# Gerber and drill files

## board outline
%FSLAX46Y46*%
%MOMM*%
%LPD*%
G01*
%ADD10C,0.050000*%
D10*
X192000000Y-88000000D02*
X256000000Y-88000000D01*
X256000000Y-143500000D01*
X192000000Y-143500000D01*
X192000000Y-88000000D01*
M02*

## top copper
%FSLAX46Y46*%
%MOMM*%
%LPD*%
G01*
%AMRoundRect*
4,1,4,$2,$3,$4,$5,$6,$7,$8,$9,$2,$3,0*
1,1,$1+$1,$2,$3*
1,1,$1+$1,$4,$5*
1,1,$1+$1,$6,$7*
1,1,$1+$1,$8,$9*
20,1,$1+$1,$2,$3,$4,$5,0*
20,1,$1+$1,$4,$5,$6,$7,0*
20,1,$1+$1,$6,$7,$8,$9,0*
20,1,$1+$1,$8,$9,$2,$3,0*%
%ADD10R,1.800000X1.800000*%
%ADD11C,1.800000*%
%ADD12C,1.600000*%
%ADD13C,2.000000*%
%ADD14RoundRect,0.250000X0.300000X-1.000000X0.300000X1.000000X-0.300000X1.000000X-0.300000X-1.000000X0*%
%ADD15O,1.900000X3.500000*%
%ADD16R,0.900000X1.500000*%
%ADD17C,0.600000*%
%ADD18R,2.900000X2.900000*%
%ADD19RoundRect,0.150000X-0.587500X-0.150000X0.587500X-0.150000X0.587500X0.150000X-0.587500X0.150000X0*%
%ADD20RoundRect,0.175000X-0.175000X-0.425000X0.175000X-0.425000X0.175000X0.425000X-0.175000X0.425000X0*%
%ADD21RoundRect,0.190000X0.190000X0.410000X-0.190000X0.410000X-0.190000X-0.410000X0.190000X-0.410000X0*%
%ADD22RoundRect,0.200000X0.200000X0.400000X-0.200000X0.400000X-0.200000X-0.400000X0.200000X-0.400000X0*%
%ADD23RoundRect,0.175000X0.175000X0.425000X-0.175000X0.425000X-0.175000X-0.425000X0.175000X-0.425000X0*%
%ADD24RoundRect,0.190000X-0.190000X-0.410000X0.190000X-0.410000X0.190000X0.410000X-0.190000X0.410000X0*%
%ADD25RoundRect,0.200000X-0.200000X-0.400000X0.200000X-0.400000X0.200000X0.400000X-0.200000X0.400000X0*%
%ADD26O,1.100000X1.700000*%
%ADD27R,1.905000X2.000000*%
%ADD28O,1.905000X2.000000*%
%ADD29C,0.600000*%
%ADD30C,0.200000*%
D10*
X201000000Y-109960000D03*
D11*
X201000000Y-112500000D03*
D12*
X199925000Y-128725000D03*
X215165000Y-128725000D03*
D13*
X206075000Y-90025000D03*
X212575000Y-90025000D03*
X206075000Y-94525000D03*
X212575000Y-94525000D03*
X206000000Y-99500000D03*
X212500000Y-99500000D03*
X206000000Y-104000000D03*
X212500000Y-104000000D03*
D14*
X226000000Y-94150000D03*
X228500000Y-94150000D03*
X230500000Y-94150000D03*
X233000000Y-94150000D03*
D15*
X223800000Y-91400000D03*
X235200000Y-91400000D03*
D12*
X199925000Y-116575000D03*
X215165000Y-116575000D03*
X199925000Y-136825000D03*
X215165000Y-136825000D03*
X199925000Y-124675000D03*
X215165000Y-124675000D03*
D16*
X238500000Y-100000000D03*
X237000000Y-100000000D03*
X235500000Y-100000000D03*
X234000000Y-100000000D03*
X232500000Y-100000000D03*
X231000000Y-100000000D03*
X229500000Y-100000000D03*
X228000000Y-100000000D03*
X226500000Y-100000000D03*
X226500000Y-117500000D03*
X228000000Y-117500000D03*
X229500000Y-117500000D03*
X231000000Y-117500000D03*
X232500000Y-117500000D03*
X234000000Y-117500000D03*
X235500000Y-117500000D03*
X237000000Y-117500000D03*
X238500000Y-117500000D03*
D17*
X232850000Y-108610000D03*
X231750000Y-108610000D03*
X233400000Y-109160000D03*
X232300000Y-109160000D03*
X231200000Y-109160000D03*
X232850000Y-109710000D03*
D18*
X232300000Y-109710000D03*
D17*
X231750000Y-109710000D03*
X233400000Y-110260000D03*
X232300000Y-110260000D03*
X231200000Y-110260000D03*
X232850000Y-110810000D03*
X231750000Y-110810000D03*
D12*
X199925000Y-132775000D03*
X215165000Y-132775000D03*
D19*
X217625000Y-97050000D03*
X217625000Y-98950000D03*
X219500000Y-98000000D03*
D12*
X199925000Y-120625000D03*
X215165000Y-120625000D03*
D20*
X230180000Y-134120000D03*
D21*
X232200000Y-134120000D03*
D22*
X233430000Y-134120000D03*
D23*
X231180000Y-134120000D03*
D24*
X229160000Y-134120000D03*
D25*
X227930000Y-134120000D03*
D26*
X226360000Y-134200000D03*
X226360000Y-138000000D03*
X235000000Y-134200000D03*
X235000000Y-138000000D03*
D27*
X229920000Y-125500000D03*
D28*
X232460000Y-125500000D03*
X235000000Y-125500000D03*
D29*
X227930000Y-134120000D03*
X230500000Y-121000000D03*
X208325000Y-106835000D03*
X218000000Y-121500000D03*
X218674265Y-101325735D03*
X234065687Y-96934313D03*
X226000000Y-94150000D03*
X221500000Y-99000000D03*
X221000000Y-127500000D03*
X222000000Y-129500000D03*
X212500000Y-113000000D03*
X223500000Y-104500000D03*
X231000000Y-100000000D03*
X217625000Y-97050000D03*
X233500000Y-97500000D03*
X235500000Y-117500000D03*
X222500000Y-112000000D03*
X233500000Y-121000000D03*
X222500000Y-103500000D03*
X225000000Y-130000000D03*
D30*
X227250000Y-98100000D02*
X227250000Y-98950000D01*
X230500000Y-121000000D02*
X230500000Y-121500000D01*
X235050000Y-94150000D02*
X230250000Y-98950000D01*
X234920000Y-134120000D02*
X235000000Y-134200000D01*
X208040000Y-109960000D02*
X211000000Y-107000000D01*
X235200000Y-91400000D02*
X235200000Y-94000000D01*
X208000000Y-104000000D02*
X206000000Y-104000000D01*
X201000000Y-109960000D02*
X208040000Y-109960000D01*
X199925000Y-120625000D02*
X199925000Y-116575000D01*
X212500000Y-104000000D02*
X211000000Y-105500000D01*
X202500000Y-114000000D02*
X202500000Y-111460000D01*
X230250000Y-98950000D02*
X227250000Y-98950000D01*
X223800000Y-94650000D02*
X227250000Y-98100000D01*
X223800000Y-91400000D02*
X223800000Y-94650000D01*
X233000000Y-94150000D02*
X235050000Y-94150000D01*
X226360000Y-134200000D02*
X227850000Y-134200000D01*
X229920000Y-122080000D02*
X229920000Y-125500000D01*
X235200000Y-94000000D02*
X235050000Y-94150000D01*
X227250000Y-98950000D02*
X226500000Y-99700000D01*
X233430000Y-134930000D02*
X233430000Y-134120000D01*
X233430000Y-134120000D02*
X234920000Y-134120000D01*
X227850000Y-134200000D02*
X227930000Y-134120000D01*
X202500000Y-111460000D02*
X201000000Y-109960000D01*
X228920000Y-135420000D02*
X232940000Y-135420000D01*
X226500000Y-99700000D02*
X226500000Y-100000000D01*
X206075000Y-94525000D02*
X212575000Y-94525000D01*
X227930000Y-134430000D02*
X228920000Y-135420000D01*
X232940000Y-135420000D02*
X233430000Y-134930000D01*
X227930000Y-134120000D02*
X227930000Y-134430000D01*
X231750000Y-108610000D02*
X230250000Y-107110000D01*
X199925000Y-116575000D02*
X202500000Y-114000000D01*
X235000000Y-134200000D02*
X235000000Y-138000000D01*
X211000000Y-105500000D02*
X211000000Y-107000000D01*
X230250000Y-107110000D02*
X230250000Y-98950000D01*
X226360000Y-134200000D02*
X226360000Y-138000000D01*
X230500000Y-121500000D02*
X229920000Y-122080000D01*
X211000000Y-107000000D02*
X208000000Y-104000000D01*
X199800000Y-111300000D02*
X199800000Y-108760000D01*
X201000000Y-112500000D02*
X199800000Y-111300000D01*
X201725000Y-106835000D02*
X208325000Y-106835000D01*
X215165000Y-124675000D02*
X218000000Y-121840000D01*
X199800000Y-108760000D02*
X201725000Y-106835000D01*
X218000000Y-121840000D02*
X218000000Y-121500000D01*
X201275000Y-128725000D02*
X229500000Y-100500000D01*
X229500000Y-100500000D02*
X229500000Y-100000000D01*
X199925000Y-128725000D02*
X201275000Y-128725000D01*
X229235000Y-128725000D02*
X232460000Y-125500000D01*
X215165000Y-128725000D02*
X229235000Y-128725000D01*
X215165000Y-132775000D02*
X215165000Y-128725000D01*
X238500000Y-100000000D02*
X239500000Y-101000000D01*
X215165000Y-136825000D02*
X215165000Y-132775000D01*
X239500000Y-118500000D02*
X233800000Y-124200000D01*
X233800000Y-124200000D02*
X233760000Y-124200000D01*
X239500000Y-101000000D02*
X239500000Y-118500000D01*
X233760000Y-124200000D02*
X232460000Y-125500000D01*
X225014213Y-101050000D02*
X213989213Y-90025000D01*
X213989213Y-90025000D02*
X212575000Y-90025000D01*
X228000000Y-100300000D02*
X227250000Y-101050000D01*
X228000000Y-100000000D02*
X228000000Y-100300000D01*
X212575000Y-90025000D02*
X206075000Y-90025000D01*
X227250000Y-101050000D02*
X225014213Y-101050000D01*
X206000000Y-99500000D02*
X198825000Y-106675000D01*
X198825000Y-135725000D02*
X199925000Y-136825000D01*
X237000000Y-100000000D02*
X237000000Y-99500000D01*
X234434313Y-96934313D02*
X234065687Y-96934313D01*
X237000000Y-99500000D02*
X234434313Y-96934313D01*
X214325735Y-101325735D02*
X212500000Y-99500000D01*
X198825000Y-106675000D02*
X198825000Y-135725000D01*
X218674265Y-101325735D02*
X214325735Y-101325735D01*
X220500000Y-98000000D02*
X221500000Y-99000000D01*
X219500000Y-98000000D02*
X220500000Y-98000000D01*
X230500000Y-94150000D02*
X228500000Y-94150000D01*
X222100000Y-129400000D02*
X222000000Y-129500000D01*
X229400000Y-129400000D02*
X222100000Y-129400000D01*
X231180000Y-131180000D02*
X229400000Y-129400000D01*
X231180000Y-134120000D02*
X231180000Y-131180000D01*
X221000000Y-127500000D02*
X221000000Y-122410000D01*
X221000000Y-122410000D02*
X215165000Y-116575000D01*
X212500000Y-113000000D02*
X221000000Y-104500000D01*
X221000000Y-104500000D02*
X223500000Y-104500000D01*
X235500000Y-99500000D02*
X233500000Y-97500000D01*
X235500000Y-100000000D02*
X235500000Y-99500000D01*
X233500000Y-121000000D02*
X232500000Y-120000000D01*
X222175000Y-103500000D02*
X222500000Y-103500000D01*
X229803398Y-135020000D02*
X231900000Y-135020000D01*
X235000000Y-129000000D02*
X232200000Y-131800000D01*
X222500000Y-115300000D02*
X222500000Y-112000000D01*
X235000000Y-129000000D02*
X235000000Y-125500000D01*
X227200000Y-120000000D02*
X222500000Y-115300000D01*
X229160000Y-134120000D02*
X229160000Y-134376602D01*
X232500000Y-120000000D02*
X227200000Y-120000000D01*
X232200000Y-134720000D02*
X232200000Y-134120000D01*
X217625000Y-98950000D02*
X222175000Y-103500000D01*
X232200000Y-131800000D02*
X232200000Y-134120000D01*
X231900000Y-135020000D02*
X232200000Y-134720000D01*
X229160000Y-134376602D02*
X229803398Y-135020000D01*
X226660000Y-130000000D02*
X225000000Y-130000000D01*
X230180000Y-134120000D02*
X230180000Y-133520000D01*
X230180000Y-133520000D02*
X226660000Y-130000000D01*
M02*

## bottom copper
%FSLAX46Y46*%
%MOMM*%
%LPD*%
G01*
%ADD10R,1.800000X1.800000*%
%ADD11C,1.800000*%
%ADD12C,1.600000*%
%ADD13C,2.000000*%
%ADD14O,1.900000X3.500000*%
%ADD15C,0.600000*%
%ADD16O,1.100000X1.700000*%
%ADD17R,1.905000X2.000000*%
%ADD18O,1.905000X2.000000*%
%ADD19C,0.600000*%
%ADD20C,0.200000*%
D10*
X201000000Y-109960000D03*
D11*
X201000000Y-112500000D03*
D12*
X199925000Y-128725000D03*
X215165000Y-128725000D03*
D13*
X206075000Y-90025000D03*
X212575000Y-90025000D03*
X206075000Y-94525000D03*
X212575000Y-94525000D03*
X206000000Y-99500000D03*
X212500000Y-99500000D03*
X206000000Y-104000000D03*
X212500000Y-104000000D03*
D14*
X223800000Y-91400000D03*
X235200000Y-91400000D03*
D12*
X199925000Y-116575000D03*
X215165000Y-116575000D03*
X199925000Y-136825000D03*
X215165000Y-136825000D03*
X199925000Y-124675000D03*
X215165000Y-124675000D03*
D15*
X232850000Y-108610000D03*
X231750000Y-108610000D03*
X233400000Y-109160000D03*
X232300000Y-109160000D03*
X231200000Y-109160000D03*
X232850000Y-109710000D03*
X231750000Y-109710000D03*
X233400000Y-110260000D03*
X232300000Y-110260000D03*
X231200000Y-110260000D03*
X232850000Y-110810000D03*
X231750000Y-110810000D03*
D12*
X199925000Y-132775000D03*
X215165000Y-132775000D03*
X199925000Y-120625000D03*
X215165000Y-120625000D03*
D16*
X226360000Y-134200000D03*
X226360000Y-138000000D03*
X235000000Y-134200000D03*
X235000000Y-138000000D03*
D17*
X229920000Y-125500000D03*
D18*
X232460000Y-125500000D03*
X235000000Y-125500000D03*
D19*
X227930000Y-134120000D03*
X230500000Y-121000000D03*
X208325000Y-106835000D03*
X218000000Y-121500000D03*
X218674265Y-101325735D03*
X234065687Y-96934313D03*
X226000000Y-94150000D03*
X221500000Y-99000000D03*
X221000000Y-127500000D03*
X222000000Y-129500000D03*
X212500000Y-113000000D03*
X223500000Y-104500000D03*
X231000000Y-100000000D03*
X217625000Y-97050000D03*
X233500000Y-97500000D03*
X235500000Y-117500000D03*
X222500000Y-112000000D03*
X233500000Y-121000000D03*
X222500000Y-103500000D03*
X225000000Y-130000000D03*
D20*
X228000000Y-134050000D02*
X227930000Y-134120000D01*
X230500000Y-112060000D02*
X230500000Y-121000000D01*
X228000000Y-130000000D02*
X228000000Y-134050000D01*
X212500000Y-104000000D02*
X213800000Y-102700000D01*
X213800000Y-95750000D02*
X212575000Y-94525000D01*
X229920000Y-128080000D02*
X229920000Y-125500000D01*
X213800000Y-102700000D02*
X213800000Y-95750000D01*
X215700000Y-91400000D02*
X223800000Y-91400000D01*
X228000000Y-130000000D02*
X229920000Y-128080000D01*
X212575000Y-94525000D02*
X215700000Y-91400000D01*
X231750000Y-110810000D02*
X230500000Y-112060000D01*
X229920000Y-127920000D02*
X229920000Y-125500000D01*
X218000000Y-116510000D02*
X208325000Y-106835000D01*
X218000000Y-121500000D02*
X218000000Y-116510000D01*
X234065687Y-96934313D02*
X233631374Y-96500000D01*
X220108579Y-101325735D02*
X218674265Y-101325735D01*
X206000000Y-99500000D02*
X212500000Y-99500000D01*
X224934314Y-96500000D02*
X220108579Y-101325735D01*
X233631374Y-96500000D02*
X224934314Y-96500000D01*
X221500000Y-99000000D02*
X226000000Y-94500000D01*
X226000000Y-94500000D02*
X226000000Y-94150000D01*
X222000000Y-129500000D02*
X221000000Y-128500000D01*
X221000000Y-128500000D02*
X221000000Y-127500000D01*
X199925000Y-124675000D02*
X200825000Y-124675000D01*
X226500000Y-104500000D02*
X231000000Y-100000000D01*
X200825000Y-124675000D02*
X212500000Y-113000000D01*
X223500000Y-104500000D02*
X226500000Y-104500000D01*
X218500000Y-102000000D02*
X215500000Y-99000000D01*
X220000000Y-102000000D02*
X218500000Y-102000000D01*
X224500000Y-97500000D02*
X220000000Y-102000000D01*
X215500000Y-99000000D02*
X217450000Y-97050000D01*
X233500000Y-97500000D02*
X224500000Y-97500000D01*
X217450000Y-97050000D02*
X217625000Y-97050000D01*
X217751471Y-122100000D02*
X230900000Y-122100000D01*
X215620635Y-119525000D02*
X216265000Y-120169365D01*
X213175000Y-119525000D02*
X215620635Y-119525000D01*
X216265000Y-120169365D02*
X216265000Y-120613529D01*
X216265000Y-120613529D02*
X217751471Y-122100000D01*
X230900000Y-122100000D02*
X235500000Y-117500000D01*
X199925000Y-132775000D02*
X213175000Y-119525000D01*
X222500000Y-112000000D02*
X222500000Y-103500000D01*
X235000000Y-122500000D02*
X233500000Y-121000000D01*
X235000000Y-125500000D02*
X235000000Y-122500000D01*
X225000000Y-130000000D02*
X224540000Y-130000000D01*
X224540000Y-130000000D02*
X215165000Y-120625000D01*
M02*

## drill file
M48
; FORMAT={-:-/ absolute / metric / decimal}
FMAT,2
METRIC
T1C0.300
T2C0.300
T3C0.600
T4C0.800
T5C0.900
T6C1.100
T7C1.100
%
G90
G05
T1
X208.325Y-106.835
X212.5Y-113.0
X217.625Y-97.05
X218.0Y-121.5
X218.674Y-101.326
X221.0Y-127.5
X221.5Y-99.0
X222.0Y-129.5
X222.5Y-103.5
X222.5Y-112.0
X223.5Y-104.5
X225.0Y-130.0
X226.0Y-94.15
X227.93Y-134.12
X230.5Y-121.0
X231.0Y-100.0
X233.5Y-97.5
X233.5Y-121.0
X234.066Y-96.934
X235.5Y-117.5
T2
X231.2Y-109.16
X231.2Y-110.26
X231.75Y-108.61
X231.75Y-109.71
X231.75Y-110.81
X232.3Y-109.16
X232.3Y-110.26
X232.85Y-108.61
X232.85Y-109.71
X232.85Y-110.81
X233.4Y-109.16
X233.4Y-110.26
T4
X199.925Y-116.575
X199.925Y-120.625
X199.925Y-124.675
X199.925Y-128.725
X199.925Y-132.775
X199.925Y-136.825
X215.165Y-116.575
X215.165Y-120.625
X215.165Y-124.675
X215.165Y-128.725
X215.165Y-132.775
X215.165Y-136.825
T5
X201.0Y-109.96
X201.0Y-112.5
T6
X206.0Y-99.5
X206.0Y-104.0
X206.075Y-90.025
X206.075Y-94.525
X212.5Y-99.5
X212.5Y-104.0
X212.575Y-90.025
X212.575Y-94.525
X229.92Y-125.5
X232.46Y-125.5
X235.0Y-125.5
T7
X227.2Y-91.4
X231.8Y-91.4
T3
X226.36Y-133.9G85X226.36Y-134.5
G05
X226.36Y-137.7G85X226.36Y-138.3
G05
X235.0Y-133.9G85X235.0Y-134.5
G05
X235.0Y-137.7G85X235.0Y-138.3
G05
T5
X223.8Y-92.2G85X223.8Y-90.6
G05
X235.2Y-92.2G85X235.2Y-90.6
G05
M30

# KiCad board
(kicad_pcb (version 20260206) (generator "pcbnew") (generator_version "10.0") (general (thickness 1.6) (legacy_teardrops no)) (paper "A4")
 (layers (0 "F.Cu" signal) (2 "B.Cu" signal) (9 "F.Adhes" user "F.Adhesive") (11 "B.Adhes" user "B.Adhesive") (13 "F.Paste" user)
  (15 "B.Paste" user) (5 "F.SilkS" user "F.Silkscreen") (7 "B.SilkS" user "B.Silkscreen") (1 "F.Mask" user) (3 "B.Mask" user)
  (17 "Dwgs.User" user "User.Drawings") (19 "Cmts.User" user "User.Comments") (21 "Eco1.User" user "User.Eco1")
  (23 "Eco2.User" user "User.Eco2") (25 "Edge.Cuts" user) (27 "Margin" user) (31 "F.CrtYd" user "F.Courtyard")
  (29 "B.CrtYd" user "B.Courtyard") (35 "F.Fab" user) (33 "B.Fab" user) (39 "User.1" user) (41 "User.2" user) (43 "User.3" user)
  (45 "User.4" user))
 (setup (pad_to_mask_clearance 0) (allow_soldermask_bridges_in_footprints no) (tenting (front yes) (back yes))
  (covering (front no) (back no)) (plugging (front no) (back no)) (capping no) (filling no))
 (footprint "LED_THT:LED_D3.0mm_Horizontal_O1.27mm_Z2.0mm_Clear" (layer "F.Cu") (at 201 109.96 -90)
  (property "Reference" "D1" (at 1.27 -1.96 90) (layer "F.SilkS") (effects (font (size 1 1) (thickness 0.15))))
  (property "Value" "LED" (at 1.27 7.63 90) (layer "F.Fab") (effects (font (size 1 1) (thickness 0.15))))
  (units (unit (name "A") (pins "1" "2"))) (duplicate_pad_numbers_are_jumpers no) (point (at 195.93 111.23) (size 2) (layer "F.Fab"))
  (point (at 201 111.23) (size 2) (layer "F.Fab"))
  (pad "1" thru_hole rect (at 0 0 270) (size 1.8 1.8) (drill 0.9) (layers "*.Cu" "*.Mask") (remove_unused_layers no) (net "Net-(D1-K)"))
  (pad "2" thru_hole circle (at 2.54 0 270) (size 1.8 1.8) (drill 0.9) (layers "*.Cu" "*.Mask") (remove_unused_layers no) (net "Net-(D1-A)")))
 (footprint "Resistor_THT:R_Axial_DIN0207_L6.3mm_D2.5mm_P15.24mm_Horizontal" (layer "F.Cu") (at 199.925 128.725)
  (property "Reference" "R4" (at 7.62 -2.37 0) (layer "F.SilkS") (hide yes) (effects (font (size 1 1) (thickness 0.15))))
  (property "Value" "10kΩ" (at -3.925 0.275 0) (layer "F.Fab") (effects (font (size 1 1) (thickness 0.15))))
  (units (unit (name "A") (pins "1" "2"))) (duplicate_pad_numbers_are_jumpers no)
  (pad "1" thru_hole circle (at 0 0) (size 1.6 1.6) (drill 0.8) (layers "*.Cu" "*.Mask") (remove_unused_layers no) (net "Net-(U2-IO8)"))
  (pad "2" thru_hole circle (at 15.24 0) (size 1.6 1.6) (drill 0.8) (layers "*.Cu" "*.Mask") (remove_unused_layers no) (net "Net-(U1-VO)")))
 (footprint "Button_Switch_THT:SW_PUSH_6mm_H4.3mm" (layer "F.Cu") (at 206.075 90.025)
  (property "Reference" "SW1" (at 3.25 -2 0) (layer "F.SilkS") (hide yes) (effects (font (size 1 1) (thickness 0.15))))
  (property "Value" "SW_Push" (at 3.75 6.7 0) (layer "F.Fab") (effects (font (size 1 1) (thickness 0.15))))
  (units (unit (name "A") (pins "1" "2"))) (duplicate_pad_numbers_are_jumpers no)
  (pad "1" thru_hole circle (at 0 0 90) (size 2 2) (drill 1.1) (layers "*.Cu" "*.Mask") (remove_unused_layers no) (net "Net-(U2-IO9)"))
  (pad "1" thru_hole circle (at 6.5 0 90) (size 2 2) (drill 1.1) (layers "*.Cu" "*.Mask") (remove_unused_layers no) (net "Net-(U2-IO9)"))
  (pad "2" thru_hole circle (at 0 4.5 90) (size 2 2) (drill 1.1) (layers "*.Cu" "*.Mask") (remove_unused_layers no) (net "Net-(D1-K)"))
  (pad "2" thru_hole circle (at 6.5 4.5 90) (size 2 2) (drill 1.1) (layers "*.Cu" "*.Mask") (remove_unused_layers no) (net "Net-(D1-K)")))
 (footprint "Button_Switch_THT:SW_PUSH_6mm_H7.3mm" (layer "F.Cu") (at 206 99.5)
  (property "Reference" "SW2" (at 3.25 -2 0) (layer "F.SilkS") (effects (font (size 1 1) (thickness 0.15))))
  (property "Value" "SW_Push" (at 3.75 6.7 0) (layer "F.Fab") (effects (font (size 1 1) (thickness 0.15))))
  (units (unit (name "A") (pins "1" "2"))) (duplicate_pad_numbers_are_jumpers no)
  (pad "1" thru_hole circle (at 0 0 90) (size 2 2) (drill 1.1) (layers "*.Cu" "*.Mask") (remove_unused_layers no) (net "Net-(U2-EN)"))
  (pad "1" thru_hole circle (at 6.5 0 90) (size 2 2) (drill 1.1) (layers "*.Cu" "*.Mask") (remove_unused_layers no) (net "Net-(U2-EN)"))
  (pad "2" thru_hole circle (at 0 4.5 90) (size 2 2) (drill 1.1) (layers "*.Cu" "*.Mask") (remove_unused_layers no) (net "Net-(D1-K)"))
  (pad "2" thru_hole circle (at 6.5 4.5 90) (size 2 2) (drill 1.1) (layers "*.Cu" "*.Mask") (remove_unused_layers no) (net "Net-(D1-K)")))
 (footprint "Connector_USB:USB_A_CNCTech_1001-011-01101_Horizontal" (layer "F.Cu") (at 229.5 84.5 90)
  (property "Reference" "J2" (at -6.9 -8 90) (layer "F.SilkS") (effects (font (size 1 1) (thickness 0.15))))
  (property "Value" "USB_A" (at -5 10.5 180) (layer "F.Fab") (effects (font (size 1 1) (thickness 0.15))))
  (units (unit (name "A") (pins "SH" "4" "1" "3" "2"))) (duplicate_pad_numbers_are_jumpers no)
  (pad "" np_thru_hole circle (at -6.9 -2.3 90) (size 1.1 1.1) (drill 1.1) (layers "*.Cu" "*.Mask"))
  (pad "" np_thru_hole circle (at -6.9 2.3 90) (size 1.1 1.1) (drill 1.1) (layers "*.Cu" "*.Mask"))
  (pad "1" smd roundrect (at -9.65 -3.5 90) (size 2.5 1.1) (layers "F.Cu" "F.Mask" "F.Paste") (roundrect_rratio 0.2272727273)
   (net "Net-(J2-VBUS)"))
  (pad "2" smd roundrect (at -9.65 -1 90) (size 2.5 1.1) (layers "F.Cu" "F.Mask" "F.Paste") (roundrect_rratio 0.2272727273)
   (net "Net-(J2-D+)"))
  (pad "3" smd roundrect (at -9.65 1 90) (size 2.5 1.1) (layers "F.Cu" "F.Mask" "F.Paste") (roundrect_rratio 0.2272727273)
   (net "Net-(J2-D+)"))
  (pad "4" smd roundrect (at -9.65 3.5 90) (size 2.5 1.1) (layers "F.Cu" "F.Mask" "F.Paste") (roundrect_rratio 0.2272727273)
   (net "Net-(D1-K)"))
  (pad "SH" thru_hole oval (at -6.9 -5.7 90) (size 3.5 1.9) (drill oval 2.5 0.9) (layers "*.Cu" "*.Mask") (remove_unused_layers no)
   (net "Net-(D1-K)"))
  (pad "SH" thru_hole oval (at -6.9 5.7 90) (size 3.5 1.9) (drill oval 2.5 0.9) (layers "*.Cu" "*.Mask") (remove_unused_layers no)
   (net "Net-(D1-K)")))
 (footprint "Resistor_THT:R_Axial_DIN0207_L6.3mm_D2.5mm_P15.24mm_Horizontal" (layer "F.Cu") (at 199.925 116.575)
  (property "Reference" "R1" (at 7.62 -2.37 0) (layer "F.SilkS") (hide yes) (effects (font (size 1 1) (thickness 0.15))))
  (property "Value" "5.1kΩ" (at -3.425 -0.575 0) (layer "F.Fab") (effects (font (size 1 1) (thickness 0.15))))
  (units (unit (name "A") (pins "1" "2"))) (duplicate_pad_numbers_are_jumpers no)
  (pad "1" thru_hole circle (at 0 0) (size 1.6 1.6) (drill 0.8) (layers "*.Cu" "*.Mask") (remove_unused_layers no) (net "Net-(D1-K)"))
  (pad "2" thru_hole circle (at 15.24 0) (size 1.6 1.6) (drill 0.8) (layers "*.Cu" "*.Mask") (remove_unused_layers no) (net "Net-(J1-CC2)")))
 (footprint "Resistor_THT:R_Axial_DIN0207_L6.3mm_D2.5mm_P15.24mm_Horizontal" (layer "F.Cu") (at 199.925 136.825)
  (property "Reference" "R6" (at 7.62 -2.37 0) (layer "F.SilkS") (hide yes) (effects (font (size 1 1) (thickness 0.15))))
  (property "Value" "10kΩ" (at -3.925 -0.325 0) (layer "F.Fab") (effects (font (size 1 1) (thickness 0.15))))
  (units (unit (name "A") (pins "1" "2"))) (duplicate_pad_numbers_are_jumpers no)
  (pad "1" thru_hole circle (at 0 0) (size 1.6 1.6) (drill 0.8) (layers "*.Cu" "*.Mask") (remove_unused_layers no) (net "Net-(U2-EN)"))
  (pad "2" thru_hole circle (at 15.24 0) (size 1.6 1.6) (drill 0.8) (layers "*.Cu" "*.Mask") (remove_unused_layers no) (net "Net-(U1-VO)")))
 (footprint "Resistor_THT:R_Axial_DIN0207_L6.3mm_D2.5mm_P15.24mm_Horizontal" (layer "F.Cu") (at 199.925 124.675)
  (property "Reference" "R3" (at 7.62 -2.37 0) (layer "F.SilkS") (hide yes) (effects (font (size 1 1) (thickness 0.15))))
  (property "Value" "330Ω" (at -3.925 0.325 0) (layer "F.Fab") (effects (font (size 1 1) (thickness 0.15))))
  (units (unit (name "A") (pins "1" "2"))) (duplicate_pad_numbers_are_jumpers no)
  (pad "1" thru_hole circle (at 0 0) (size 1.6 1.6) (drill 0.8) (layers "*.Cu" "*.Mask") (remove_unused_layers no) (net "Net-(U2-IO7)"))
  (pad "2" thru_hole circle (at 15.24 0) (size 1.6 1.6) (drill 0.8) (layers "*.Cu" "*.Mask") (remove_unused_layers no) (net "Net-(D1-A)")))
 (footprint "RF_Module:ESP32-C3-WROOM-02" (layer "F.Cu") (at 232.5 108.75 -90)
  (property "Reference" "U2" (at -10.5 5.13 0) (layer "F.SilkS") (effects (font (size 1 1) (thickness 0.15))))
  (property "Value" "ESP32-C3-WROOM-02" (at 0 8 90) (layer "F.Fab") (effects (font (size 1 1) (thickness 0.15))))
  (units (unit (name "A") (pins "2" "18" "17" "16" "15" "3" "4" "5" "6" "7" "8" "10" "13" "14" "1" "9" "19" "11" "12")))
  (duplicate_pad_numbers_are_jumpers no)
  (pad "" smd rect (at -0.14 -0.9 270) (size 0.7 0.7) (layers "F.Paste"))
  (pad "" smd rect (at -0.14 0.2 270) (size 0.7 0.7) (layers "F.Paste"))
  (pad "" smd rect (at -0.14 1.3 270) (size 0.7 0.7) (layers "F.Paste"))
  (pad "" smd rect (at 0.96 -0.9 270) (size 0.7 0.7) (layers "F.Paste"))
  (pad "" smd rect (at 0.96 0.2 270) (size 0.7 0.7) (layers "F.Paste"))
  (pad "" smd rect (at 0.96 1.3 270) (size 0.7 0.7) (layers "F.Paste"))
  (pad "" smd rect (at 2.06 -0.9 270) (size 0.7 0.7) (layers "F.Paste"))
  (pad "" smd rect (at 2.06 0.2 270) (size 0.7 0.7) (layers "F.Paste"))
  (pad "" smd rect (at 2.06 1.3 270) (size 0.7 0.7) (layers "F.Paste"))
  (pad "1" smd rect (at -8.75 -6 270) (size 1.5 0.9) (layers "F.Cu" "F.Mask" "F.Paste") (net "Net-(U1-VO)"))
  (pad "2" smd rect (at -8.75 -4.5 270) (size 1.5 0.9) (layers "F.Cu" "F.Mask" "F.Paste") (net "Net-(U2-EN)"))
  (pad "3" smd rect (at -8.75 -3 270) (size 1.5 0.9) (layers "F.Cu" "F.Mask" "F.Paste") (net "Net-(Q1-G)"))
  (pad "4" smd rect (at -8.75 -1.5 270) (size 1.5 0.9) (layers "F.Cu" "F.Mask" "F.Paste") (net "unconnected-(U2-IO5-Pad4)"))
  (pad "5" smd rect (at -8.75 0 270) (size 1.5 0.9) (layers "F.Cu" "F.Mask" "F.Paste") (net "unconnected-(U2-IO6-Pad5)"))
  (pad "6" smd rect (at -8.75 1.5 270) (size 1.5 0.9) (layers "F.Cu" "F.Mask" "F.Paste") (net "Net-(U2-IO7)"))
  (pad "7" smd rect (at -8.75 3 270) (size 1.5 0.9) (layers "F.Cu" "F.Mask" "F.Paste") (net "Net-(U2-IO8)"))
  (pad "8" smd rect (at -8.75 4.5 270) (size 1.5 0.9) (layers "F.Cu" "F.Mask" "F.Paste") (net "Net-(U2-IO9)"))
  (pad "9" smd rect (at -8.75 6 270) (size 1.5 0.9) (layers "F.Cu" "F.Mask" "F.Paste") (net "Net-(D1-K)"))
  (pad "10" smd rect (at 8.75 6 270) (size 1.5 0.9) (layers "F.Cu" "F.Mask" "F.Paste") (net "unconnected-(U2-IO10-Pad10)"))
  (pad "11" smd rect (at 8.75 4.5 270) (size 1.5 0.9) (layers "F.Cu" "F.Mask" "F.Paste") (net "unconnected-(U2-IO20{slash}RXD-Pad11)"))
  (pad "12" smd rect (at 8.75 3 270) (size 1.5 0.9) (layers "F.Cu" "F.Mask" "F.Paste") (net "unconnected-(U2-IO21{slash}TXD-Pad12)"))
  (pad "13" smd rect (at 8.75 1.5 270) (size 1.5 0.9) (layers "F.Cu" "F.Mask" "F.Paste") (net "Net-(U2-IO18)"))
  (pad "14" smd rect (at 8.75 0 270) (size 1.5 0.9) (layers "F.Cu" "F.Mask" "F.Paste") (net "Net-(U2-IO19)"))
  (pad "15" smd rect (at 8.75 -1.5 270) (size 1.5 0.9) (layers "F.Cu" "F.Mask" "F.Paste") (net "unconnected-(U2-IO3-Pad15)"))
  (pad "16" smd rect (at 8.75 -3 270) (size 1.5 0.9) (layers "F.Cu" "F.Mask" "F.Paste") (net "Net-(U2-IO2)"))
  (pad "17" smd rect (at 8.75 -4.5 270) (size 1.5 0.9) (layers "F.Cu" "F.Mask" "F.Paste") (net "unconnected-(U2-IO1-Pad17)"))
  (pad "18" smd rect (at 8.75 -6 270) (size 1.5 0.9) (layers "F.Cu" "F.Mask" "F.Paste") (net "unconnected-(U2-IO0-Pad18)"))
  (pad "19" thru_hole circle (at -0.14 -0.35 270) (size 0.6 0.6) (drill 0.3) (layers "*.Cu" "F.Mask") (remove_unused_layers no)
   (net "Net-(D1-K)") (zone_connect 2))
  (pad "19" thru_hole circle (at -0.14 0.75 270) (size 0.6 0.6) (drill 0.3) (layers "*.Cu" "F.Mask") (remove_unused_layers no)
   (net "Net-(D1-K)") (zone_connect 2))
  (pad "19" thru_hole circle (at 0.41 -0.9 270) (size 0.6 0.6) (drill 0.3) (layers "*.Cu" "F.Mask") (remove_unused_layers no)
   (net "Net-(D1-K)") (zone_connect 2))
  (pad "19" thru_hole circle (at 0.41 0.2 270) (size 0.6 0.6) (drill 0.3) (layers "*.Cu" "F.Mask") (remove_unused_layers no)
   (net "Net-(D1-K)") (zone_connect 2))
  (pad "19" thru_hole circle (at 0.41 1.3 270) (size 0.6 0.6) (drill 0.3) (layers "*.Cu" "F.Mask") (remove_unused_layers no)
   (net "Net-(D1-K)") (zone_connect 2))
  (pad "19" thru_hole circle (at 0.96 -0.35 270) (size 0.6 0.6) (drill 0.3) (layers "*.Cu" "F.Mask") (remove_unused_layers no)
   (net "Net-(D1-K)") (zone_connect 2))
  (pad "19" smd rect (at 0.96 0.2 270) (size 2.9 2.9) (layers "F.Cu" "F.Mask") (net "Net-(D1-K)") (zone_connect 2))
  (pad "19" thru_hole circle (at 0.96 0.75 270) (size 0.6 0.6) (drill 0.3) (layers "*.Cu" "F.Mask") (remove_unused_layers no)
   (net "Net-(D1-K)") (zone_connect 2))
  (pad "19" thru_hole circle (at 1.51 -0.9 270) (size 0.6 0.6) (drill 0.3) (layers "*.Cu" "F.Mask") (remove_unused_layers no)
   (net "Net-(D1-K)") (zone_connect 2))
  (pad "19" thru_hole circle (at 1.51 0.2 270) (size 0.6 0.6) (drill 0.3) (layers "*.Cu" "F.Mask") (remove_unused_layers no)
   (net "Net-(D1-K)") (zone_connect 2))
  (pad "19" thru_hole circle (at 1.51 1.3 270) (size 0.6 0.6) (drill 0.3) (layers "*.Cu" "F.Mask") (remove_unused_layers no)
   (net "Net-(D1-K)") (zone_connect 2))
  (pad "19" thru_hole circle (at 2.06 -0.35 270) (size 0.6 0.6) (drill 0.3) (layers "*.Cu" "F.Mask") (remove_unused_layers no)
   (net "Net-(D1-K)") (zone_connect 2))
  (pad "19" thru_hole circle (at 2.06 0.75 270) (size 0.6 0.6) (drill 0.3) (layers "*.Cu" "F.Mask") (remove_unused_layers no)
   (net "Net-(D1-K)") (zone_connect 2))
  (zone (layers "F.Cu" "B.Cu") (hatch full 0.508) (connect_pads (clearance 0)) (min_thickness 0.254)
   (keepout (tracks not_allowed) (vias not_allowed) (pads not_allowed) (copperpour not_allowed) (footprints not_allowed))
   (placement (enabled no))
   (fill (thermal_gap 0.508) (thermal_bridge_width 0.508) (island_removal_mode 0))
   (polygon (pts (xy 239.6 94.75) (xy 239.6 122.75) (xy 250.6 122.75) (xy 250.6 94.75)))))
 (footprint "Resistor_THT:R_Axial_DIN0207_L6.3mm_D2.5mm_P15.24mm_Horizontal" (layer "F.Cu") (at 199.925 132.775)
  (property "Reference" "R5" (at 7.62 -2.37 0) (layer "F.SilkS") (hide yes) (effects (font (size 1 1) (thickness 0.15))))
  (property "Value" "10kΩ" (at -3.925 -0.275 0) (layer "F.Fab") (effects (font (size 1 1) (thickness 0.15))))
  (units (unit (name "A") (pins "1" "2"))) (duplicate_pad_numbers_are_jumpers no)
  (pad "1" thru_hole circle (at 0 0) (size 1.6 1.6) (drill 0.8) (layers "*.Cu" "*.Mask") (remove_unused_layers no) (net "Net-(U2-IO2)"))
  (pad "2" thru_hole circle (at 15.24 0) (size 1.6 1.6) (drill 0.8) (layers "*.Cu" "*.Mask") (remove_unused_layers no) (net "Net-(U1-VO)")))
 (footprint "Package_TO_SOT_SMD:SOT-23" (layer "F.Cu") (at 218.5625 98)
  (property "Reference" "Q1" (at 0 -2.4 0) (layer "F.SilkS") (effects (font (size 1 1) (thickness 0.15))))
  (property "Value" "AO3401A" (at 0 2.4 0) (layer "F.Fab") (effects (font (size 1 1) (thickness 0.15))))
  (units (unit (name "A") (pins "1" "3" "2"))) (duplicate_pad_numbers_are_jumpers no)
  (pad "1" smd roundrect (at -0.9375 -0.95) (size 1.475 0.6) (layers "F.Cu" "F.Mask" "F.Paste") (roundrect_rratio 0.25) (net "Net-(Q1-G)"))
  (pad "2" smd roundrect (at -0.9375 0.95) (size 1.475 0.6) (layers "F.Cu" "F.Mask" "F.Paste") (roundrect_rratio 0.25) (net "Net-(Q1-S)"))
  (pad "3" smd roundrect (at 0.9375 0) (size 1.475 0.6) (layers "F.Cu" "F.Mask" "F.Paste") (roundrect_rratio 0.25) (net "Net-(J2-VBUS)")))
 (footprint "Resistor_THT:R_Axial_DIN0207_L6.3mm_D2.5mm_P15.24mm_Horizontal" (layer "F.Cu") (at 199.925 120.625)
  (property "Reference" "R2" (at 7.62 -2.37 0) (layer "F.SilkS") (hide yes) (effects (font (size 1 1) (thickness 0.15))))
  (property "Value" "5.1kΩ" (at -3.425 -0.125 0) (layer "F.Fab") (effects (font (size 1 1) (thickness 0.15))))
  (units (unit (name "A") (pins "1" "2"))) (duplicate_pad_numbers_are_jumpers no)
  (pad "1" thru_hole circle (at 0 0) (size 1.6 1.6) (drill 0.8) (layers "*.Cu" "*.Mask") (remove_unused_layers no) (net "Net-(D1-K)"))
  (pad "2" thru_hole circle (at 15.24 0) (size 1.6 1.6) (drill 0.8) (layers "*.Cu" "*.Mask") (remove_unused_layers no) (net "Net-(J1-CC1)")))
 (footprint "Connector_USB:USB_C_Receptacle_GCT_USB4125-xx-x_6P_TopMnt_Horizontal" (layer "F.Cu") (at 230.68 137.2)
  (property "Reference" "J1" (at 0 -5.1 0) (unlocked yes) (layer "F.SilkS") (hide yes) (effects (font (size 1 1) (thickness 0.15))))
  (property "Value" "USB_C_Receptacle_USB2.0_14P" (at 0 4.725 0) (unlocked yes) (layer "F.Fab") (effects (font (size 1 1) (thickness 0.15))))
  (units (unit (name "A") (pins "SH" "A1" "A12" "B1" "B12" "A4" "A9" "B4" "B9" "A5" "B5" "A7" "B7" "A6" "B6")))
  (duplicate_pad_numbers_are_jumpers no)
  (pad "A5" smd roundrect (at -0.5 -3.08) (size 0.7 1.2) (layers "F.Cu" "F.Mask" "F.Paste") (roundrect_rratio 0.25) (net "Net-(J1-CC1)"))
  (pad "A9" smd roundrect (at 1.52 -3.08 180) (size 0.76 1.2) (layers "F.Cu" "F.Mask" "F.Paste") (roundrect_rratio 0.25) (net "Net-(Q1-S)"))
  (pad "A12" smd roundrect (at 2.75 -3.08 180) (size 0.8 1.2) (layers "F.Cu" "F.Mask" "F.Paste") (roundrect_rratio 0.25) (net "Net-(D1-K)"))
  (pad "B5" smd roundrect (at 0.5 -3.08 180) (size 0.7 1.2) (layers "F.Cu" "F.Mask" "F.Paste") (roundrect_rratio 0.25) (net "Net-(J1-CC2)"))
  (pad "B9" smd roundrect (at -1.52 -3.08) (size 0.76 1.2) (layers "F.Cu" "F.Mask" "F.Paste") (roundrect_rratio 0.25) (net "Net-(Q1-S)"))
  (pad "B12" smd roundrect (at -2.75 -3.08) (size 0.8 1.2) (layers "F.Cu" "F.Mask" "F.Paste") (roundrect_rratio 0.25) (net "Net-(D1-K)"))
  (pad "SH" thru_hole oval (at -4.32 -3) (size 1.1 1.7) (drill oval 0.6 1.2) (layers "*.Cu" "*.Mask" "F.Paste") (remove_unused_layers no)
   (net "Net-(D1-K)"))
  (pad "SH" thru_hole oval (at -4.32 0.8) (size 1.1 1.7) (drill oval 0.6 1.2) (layers "*.Cu" "*.Mask" "F.Paste") (remove_unused_layers no)
   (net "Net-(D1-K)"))
  (pad "SH" thru_hole oval (at 4.32 -3) (size 1.1 1.7) (drill oval 0.6 1.2) (layers "*.Cu" "*.Mask" "F.Paste") (remove_unused_layers no)
   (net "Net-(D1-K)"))
  (pad "SH" thru_hole oval (at 4.32 0.8) (size 1.1 1.7) (drill oval 0.6 1.2) (layers "*.Cu" "*.Mask" "F.Paste") (remove_unused_layers no)
   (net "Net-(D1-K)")))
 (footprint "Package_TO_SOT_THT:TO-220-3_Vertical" (layer "F.Cu") (at 229.92 125.5)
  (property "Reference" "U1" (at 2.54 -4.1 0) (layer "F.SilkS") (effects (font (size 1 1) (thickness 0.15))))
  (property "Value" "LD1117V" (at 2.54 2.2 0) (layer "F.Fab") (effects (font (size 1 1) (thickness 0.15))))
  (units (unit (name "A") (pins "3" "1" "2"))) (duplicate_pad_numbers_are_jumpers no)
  (pad "1" thru_hole rect (at 0 0) (size 1.905 2) (drill 1.1) (layers "*.Cu" "*.Mask") (remove_unused_layers no) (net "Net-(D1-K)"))
  (pad "2" thru_hole oval (at 2.54 0) (size 1.905 2) (drill 1.1) (layers "*.Cu" "*.Mask") (remove_unused_layers no) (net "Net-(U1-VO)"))
  (pad "3" thru_hole oval (at 5.08 0) (size 1.905 2) (drill 1.1) (layers "*.Cu" "*.Mask") (remove_unused_layers no) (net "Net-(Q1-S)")))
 (gr_rect (start 192 88) (end 256 143.5) (stroke (width 0.05) (type default)) (fill no) (layer "Edge.Cuts"))
 (segment (start 227.25 98.1) (end 227.25 98.95) (width 0.2) (layer "F.Cu") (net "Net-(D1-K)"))
 (segment (start 230.5 121) (end 230.5 121.5) (width 0.2) (layer "F.Cu") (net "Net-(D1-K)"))
 (segment (start 235.05 94.15) (end 230.25 98.95) (width 0.2) (layer "F.Cu") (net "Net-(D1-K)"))
 (segment (start 234.92 134.12) (end 235 134.2) (width 0.2) (layer "F.Cu") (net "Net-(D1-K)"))
 (segment (start 208.04 109.96) (end 211 107) (width 0.2) (layer "F.Cu") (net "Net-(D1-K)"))
 (segment (start 235.2 91.4) (end 235.2 94) (width 0.2) (layer "F.Cu") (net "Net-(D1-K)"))
 (segment (start 208 104) (end 206 104) (width 0.2) (layer "F.Cu") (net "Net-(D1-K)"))
 (segment (start 201 109.96) (end 208.04 109.96) (width 0.2) (layer "F.Cu") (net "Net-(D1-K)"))
 (segment (start 199.925 120.625) (end 199.925 116.575) (width 0.2) (layer "F.Cu") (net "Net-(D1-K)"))
 (segment (start 212.5 104) (end 211 105.5) (width 0.2) (layer "F.Cu") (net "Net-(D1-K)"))
 (segment (start 202.5 114) (end 202.5 111.46) (width 0.2) (layer "F.Cu") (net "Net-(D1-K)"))
 (segment (start 230.25 98.95) (end 227.25 98.95) (width 0.2) (layer "F.Cu") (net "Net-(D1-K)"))
 (segment (start 223.8 94.65) (end 227.25 98.1) (width 0.2) (layer "F.Cu") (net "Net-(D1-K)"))
 (segment (start 223.8 91.4) (end 223.8 94.65) (width 0.2) (layer "F.Cu") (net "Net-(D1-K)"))
 (segment (start 233 94.15) (end 235.05 94.15) (width 0.2) (layer "F.Cu") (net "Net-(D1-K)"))
 (segment (start 226.36 134.2) (end 227.85 134.2) (width 0.2) (layer "F.Cu") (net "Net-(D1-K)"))
 (segment (start 229.92 122.08) (end 229.92 125.5) (width 0.2) (layer "F.Cu") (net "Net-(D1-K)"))
 (segment (start 235.2 94) (end 235.05 94.15) (width 0.2) (layer "F.Cu") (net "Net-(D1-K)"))
 (segment (start 227.25 98.95) (end 226.5 99.7) (width 0.2) (layer "F.Cu") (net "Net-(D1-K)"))
 (segment (start 233.43 134.93) (end 233.43 134.12) (width 0.2) (layer "F.Cu") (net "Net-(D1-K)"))
 (segment (start 233.43 134.12) (end 234.92 134.12) (width 0.2) (layer "F.Cu") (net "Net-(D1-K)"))
 (segment (start 227.85 134.2) (end 227.93 134.12) (width 0.2) (layer "F.Cu") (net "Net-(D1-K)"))
 (segment (start 202.5 111.46) (end 201 109.96) (width 0.2) (layer "F.Cu") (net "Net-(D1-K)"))
 (segment (start 228.92 135.42) (end 232.94 135.42) (width 0.2) (layer "F.Cu") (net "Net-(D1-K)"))
 (segment (start 226.5 99.7) (end 226.5 100) (width 0.2) (layer "F.Cu") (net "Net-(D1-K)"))
 (segment (start 206.075 94.525) (end 212.575 94.525) (width 0.2) (layer "F.Cu") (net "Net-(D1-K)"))
 (segment (start 227.93 134.43) (end 228.92 135.42) (width 0.2) (layer "F.Cu") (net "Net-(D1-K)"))
 (segment (start 232.94 135.42) (end 233.43 134.93) (width 0.2) (layer "F.Cu") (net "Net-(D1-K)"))
 (segment (start 227.93 134.12) (end 227.93 134.43) (width 0.2) (layer "F.Cu") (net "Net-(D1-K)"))
 (segment (start 231.75 108.61) (end 230.25 107.11) (width 0.2) (layer "F.Cu") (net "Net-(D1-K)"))
 (segment (start 199.925 116.575) (end 202.5 114) (width 0.2) (layer "F.Cu") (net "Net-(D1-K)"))
 (segment (start 235 134.2) (end 235 138) (width 0.2) (layer "F.Cu") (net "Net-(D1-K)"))
 (segment (start 211 105.5) (end 211 107) (width 0.2) (layer "F.Cu") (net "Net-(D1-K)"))
 (segment (start 230.25 107.11) (end 230.25 98.95) (width 0.2) (layer "F.Cu") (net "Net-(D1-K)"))
 (segment (start 226.36 134.2) (end 226.36 138) (width 0.2) (layer "F.Cu") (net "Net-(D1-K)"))
 (segment (start 230.5 121.5) (end 229.92 122.08) (width 0.2) (layer "F.Cu") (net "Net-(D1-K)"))
 (segment (start 211 107) (end 208 104) (width 0.2) (layer "F.Cu") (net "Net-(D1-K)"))
 (via (at 227.93 134.12) (size 0.6) (drill 0.3) (layers "F.Cu" "B.Cu") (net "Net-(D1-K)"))
 (via (at 230.5 121) (size 0.6) (drill 0.3) (layers "F.Cu" "B.Cu") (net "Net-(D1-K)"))
 (segment (start 228 134.05) (end 227.93 134.12) (width 0.2) (layer "B.Cu") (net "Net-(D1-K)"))
 (segment (start 230.5 112.06) (end 230.5 121) (width 0.2) (layer "B.Cu") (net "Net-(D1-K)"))
 (segment (start 228 130) (end 228 134.05) (width 0.2) (layer "B.Cu") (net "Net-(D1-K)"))
 (segment (start 212.5 104) (end 213.8 102.7) (width 0.2) (layer "B.Cu") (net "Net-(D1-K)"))
 (segment (start 213.8 95.75) (end 212.575 94.525) (width 0.2) (layer "B.Cu") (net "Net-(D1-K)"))
 (segment (start 229.92 128.08) (end 229.92 125.5) (width 0.2) (layer "B.Cu") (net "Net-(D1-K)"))
 (segment (start 213.8 102.7) (end 213.8 95.75) (width 0.2) (layer "B.Cu") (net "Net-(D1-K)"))
 (segment (start 215.7 91.4) (end 223.8 91.4) (width 0.2) (layer "B.Cu") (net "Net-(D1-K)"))
 (segment (start 228 130) (end 229.92 128.08) (width 0.2) (layer "B.Cu") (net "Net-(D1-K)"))
 (segment (start 212.575 94.525) (end 215.7 91.4) (width 0.2) (layer "B.Cu") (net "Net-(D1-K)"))
 (segment (start 231.75 110.81) (end 230.5 112.06) (width 0.2) (layer "B.Cu") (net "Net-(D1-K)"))
 (segment (start 229.92 127.92) (end 229.92 125.5) (width 0.2) (layer "B.Cu") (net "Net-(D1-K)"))
 (segment (start 199.8 111.3) (end 199.8 108.76) (width 0.2) (layer "F.Cu") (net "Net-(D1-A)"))
 (segment (start 201 112.5) (end 199.8 111.3) (width 0.2) (layer "F.Cu") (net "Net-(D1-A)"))
 (segment (start 201.725 106.835) (end 208.325 106.835) (width 0.2) (layer "F.Cu") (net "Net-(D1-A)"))
 (segment (start 215.165 124.675) (end 218 121.84) (width 0.2) (layer "F.Cu") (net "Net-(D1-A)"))
 (segment (start 199.8 108.76) (end 201.725 106.835) (width 0.2) (layer "F.Cu") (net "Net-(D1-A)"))
 (segment (start 218 121.84) (end 218 121.5) (width 0.2) (layer "F.Cu") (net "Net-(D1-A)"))
 (via (at 208.325 106.835) (size 0.6) (drill 0.3) (layers "F.Cu" "B.Cu") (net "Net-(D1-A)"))
 (via (at 218 121.5) (size 0.6) (drill 0.3) (layers "F.Cu" "B.Cu") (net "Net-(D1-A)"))
 (segment (start 218 116.51) (end 208.325 106.835) (width 0.2) (layer "B.Cu") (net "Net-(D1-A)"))
 (segment (start 218 121.5) (end 218 116.51) (width 0.2) (layer "B.Cu") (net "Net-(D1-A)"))
 (segment (start 201.275 128.725) (end 229.5 100.5) (width 0.2) (layer "F.Cu") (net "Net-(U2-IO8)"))
 (segment (start 229.5 100.5) (end 229.5 100) (width 0.2) (layer "F.Cu") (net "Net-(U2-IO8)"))
 (segment (start 199.925 128.725) (end 201.275 128.725) (width 0.2) (layer "F.Cu") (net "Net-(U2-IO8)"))
 (segment (start 229.235 128.725) (end 232.46 125.5) (width 0.2) (layer "F.Cu") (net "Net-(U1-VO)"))
 (segment (start 215.165 128.725) (end 229.235 128.725) (width 0.2) (layer "F.Cu") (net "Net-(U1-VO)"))
 (segment (start 215.165 132.775) (end 215.165 128.725) (width 0.2) (layer "F.Cu") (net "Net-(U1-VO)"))
 (segment (start 238.5 100) (end 239.5 101) (width 0.2) (layer "F.Cu") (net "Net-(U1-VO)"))
 (segment (start 215.165 136.825) (end 215.165 132.775) (width 0.2) (layer "F.Cu") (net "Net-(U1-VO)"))
 (segment (start 239.5 118.5) (end 233.8 124.2) (width 0.2) (layer "F.Cu") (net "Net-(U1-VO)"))
 (segment (start 233.8 124.2) (end 233.76 124.2) (width 0.2) (layer "F.Cu") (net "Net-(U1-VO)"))
 (segment (start 239.5 101) (end 239.5 118.5) (width 0.2) (layer "F.Cu") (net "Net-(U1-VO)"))
 (segment (start 233.76 124.2) (end 232.46 125.5) (width 0.2) (layer "F.Cu") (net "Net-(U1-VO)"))
 (segment (start 225.014213 101.05) (end 213.989213 90.025) (width 0.2) (layer "F.Cu") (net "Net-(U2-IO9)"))
 (segment (start 213.989213 90.025) (end 212.575 90.025) (width 0.2) (layer "F.Cu") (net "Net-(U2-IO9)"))
 (segment (start 228 100.3) (end 227.25 101.05) (width 0.2) (layer "F.Cu") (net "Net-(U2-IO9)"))
 (segment (start 228 100) (end 228 100.3) (width 0.2) (layer "F.Cu") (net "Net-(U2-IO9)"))
 (segment (start 212.575 90.025) (end 206.075 90.025) (width 0.2) (layer "F.Cu") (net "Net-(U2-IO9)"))
 (segment (start 227.25 101.05) (end 225.014213 101.05) (width 0.2) (layer "F.Cu") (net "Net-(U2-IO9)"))
 (segment (start 206 99.5) (end 198.825 106.675) (width 0.2) (layer "F.Cu") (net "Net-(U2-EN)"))
 (segment (start 198.825 135.725) (end 199.925 136.825) (width 0.2) (layer "F.Cu") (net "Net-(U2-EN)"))
 (segment (start 237 100) (end 237 99.5) (width 0.2) (layer "F.Cu") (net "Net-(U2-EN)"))
 (segment (start 234.434313 96.934313) (end 234.065687 96.934313) (width 0.2) (layer "F.Cu") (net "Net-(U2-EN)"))
 (segment (start 237 99.5) (end 234.434313 96.934313) (width 0.2) (layer "F.Cu") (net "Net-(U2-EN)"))
 (segment (start 214.325735 101.325735) (end 212.5 99.5) (width 0.2) (layer "F.Cu") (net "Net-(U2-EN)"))
 (segment (start 198.825 106.675) (end 198.825 135.725) (width 0.2) (layer "F.Cu") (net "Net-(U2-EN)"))
 (segment (start 218.674265 101.325735) (end 214.325735 101.325735) (width 0.2) (layer "F.Cu") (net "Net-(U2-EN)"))
 (via (at 218.674265 101.325735) (size 0.6) (drill 0.3) (layers "F.Cu" "B.Cu") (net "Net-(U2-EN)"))
 (via (at 234.065687 96.934313) (size 0.6) (drill 0.3) (layers "F.Cu" "B.Cu") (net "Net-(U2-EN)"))
 (segment (start 234.065687 96.934313) (end 233.631374 96.5) (width 0.2) (layer "B.Cu") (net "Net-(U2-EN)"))
 (segment (start 220.108579 101.325735) (end 218.674265 101.325735) (width 0.2) (layer "B.Cu") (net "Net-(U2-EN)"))
 (segment (start 206 99.5) (end 212.5 99.5) (width 0.2) (layer "B.Cu") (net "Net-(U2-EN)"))
 (segment (start 224.934314 96.5) (end 220.108579 101.325735) (width 0.2) (layer "B.Cu") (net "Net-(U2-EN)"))
 (segment (start 233.631374 96.5) (end 224.934314 96.5) (width 0.2) (layer "B.Cu") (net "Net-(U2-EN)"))
 (segment (start 220.5 98) (end 221.5 99) (width 0.2) (layer "F.Cu") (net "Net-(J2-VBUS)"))
 (segment (start 219.5 98) (end 220.5 98) (width 0.2) (layer "F.Cu") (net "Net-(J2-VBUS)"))
 (via (at 226 94.15) (size 0.6) (drill 0.3) (layers "F.Cu" "B.Cu") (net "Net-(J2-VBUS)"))
 (via (at 221.5 99) (size 0.6) (drill 0.3) (layers "F.Cu" "B.Cu") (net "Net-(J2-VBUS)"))
 (segment (start 221.5 99) (end 226 94.5) (width 0.2) (layer "B.Cu") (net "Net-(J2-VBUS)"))
 (segment (start 226 94.5) (end 226 94.15) (width 0.2) (layer "B.Cu") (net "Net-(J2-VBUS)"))
 (segment (start 230.5 94.15) (end 228.5 94.15) (width 0.2) (layer "F.Cu") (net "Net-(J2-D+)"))
 (segment (start 222.1 129.4) (end 222 129.5) (width 0.2) (layer "F.Cu") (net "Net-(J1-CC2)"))
 (segment (start 229.4 129.4) (end 222.1 129.4) (width 0.2) (layer "F.Cu") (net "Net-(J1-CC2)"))
 (segment (start 231.18 131.18) (end 229.4 129.4) (width 0.2) (layer "F.Cu") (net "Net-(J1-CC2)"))
 (segment (start 231.18 134.12) (end 231.18 131.18) (width 0.2) (layer "F.Cu") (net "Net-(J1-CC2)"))
 (segment (start 221 127.5) (end 221 122.41) (width 0.2) (layer "F.Cu") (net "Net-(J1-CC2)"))
 (segment (start 221 122.41) (end 215.165 116.575) (width 0.2) (layer "F.Cu") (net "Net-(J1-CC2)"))
 (via (at 221 127.5) (size 0.6) (drill 0.3) (layers "F.Cu" "B.Cu") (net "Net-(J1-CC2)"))
 (via (at 222 129.5) (size 0.6) (drill 0.3) (layers "F.Cu" "B.Cu") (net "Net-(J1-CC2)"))
 (segment (start 222 129.5) (end 221 128.5) (width 0.2) (layer "B.Cu") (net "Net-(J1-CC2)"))
 (segment (start 221 128.5) (end 221 127.5) (width 0.2) (layer "B.Cu") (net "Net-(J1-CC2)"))
 (segment (start 212.5 113) (end 221 104.5) (width 0.2) (layer "F.Cu") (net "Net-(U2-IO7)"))
 (segment (start 221 104.5) (end 223.5 104.5) (width 0.2) (layer "F.Cu") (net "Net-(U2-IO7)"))
 (via (at 212.5 113) (size 0.6) (drill 0.3) (layers "F.Cu" "B.Cu") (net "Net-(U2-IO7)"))
 (via (at 223.5 104.5) (size 0.6) (drill 0.3) (layers "F.Cu" "B.Cu") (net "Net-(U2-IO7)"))
 (via (at 231 100) (size 0.6) (drill 0.3) (layers "F.Cu" "B.Cu") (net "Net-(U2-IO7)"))
 (segment (start 199.925 124.675) (end 200.825 124.675) (width 0.2) (layer "B.Cu") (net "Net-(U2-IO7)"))
 (segment (start 226.5 104.5) (end 231 100) (width 0.2) (layer "B.Cu") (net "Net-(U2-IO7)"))
 (segment (start 200.825 124.675) (end 212.5 113) (width 0.2) (layer "B.Cu") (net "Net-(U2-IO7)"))
 (segment (start 223.5 104.5) (end 226.5 104.5) (width 0.2) (layer "B.Cu") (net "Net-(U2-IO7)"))
 (segment (start 235.5 99.5) (end 233.5 97.5) (width 0.2) (layer "F.Cu") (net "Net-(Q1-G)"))
 (segment (start 235.5 100) (end 235.5 99.5) (width 0.2) (layer "F.Cu") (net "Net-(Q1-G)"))
 (via (at 217.625 97.05) (size 0.6) (drill 0.3) (layers "F.Cu" "B.Cu") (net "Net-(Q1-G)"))
 (via (at 233.5 97.5) (size 0.6) (drill 0.3) (layers "F.Cu" "B.Cu") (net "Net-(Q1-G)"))
 (segment (start 218.5 102) (end 215.5 99) (width 0.2) (layer "B.Cu") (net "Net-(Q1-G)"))
 (segment (start 220 102) (end 218.5 102) (width 0.2) (layer "B.Cu") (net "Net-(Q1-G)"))
 (segment (start 224.5 97.5) (end 220 102) (width 0.2) (layer "B.Cu") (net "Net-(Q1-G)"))
 (segment (start 215.5 99) (end 217.45 97.05) (width 0.2) (layer "B.Cu") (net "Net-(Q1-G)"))
 (segment (start 233.5 97.5) (end 224.5 97.5) (width 0.2) (layer "B.Cu") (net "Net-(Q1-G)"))
 (segment (start 217.45 97.05) (end 217.625 97.05) (width 0.2) (layer "B.Cu") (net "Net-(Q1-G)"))
 (via (at 235.5 117.5) (size 0.6) (drill 0.3) (layers "F.Cu" "B.Cu") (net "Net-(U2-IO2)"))
 (segment (start 217.751471 122.1) (end 230.9 122.1) (width 0.2) (layer "B.Cu") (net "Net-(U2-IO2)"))
 (segment (start 215.620635 119.525) (end 216.265 120.169365) (width 0.2) (layer "B.Cu") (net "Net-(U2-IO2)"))
 (segment (start 213.175 119.525) (end 215.620635 119.525) (width 0.2) (layer "B.Cu") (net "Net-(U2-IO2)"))
 (segment (start 216.265 120.169365) (end 216.265 120.613529) (width 0.2) (layer "B.Cu") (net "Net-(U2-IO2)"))
 (segment (start 216.265 120.613529) (end 217.751471 122.1) (width 0.2) (layer "B.Cu") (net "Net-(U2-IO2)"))
 (segment (start 230.9 122.1) (end 235.5 117.5) (width 0.2) (layer "B.Cu") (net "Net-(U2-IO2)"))
 (segment (start 199.925 132.775) (end 213.175 119.525) (width 0.2) (layer "B.Cu") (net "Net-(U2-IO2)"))
 (segment (start 233.5 121) (end 232.5 120) (width 0.2) (layer "F.Cu") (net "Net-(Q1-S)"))
 (segment (start 222.175 103.5) (end 222.5 103.5) (width 0.2) (layer "F.Cu") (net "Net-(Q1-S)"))
 (segment (start 229.803398 135.02) (end 231.9 135.02) (width 0.2) (layer "F.Cu") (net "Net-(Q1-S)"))
 (segment (start 235 129) (end 232.2 131.8) (width 0.2) (layer "F.Cu") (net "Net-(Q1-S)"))
 (segment (start 222.5 115.3) (end 222.5 112) (width 0.2) (layer "F.Cu") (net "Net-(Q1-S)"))
 (segment (start 235 129) (end 235 125.5) (width 0.2) (layer "F.Cu") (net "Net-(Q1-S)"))
 (segment (start 227.2 120) (end 222.5 115.3) (width 0.2) (layer "F.Cu") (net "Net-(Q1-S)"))
 (segment (start 229.16 134.12) (end 229.16 134.376602) (width 0.2) (layer "F.Cu") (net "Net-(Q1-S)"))
 (segment (start 232.5 120) (end 227.2 120) (width 0.2) (layer "F.Cu") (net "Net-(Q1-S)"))
 (segment (start 232.2 134.72) (end 232.2 134.12) (width 0.2) (layer "F.Cu") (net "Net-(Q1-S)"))
 (segment (start 217.625 98.95) (end 222.175 103.5) (width 0.2) (layer "F.Cu") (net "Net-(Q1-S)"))
 (segment (start 232.2 131.8) (end 232.2 134.12) (width 0.2) (layer "F.Cu") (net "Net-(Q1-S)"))
 (segment (start 231.9 135.02) (end 232.2 134.72) (width 0.2) (layer "F.Cu") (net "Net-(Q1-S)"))
 (segment (start 229.16 134.376602) (end 229.803398 135.02) (width 0.2) (layer "F.Cu") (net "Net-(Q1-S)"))
 (via (at 222.5 112) (size 0.6) (drill 0.3) (layers "F.Cu" "B.Cu") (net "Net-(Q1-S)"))
 (via (at 233.5 121) (size 0.6) (drill 0.3) (layers "F.Cu" "B.Cu") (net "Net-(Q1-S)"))
 (via (at 222.5 103.5) (size 0.6) (drill 0.3) (layers "F.Cu" "B.Cu") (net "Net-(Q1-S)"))
 (segment (start 222.5 112) (end 222.5 103.5) (width 0.2) (layer "B.Cu") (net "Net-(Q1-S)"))
 (segment (start 235 122.5) (end 233.5 121) (width 0.2) (layer "B.Cu") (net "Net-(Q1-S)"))
 (segment (start 235 125.5) (end 235 122.5) (width 0.2) (layer "B.Cu") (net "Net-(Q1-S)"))
 (segment (start 226.66 130) (end 225 130) (width 0.2) (layer "F.Cu") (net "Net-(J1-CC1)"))
 (segment (start 230.18 134.12) (end 230.18 133.52) (width 0.2) (layer "F.Cu") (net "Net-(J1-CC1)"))
 (segment (start 230.18 133.52) (end 226.66 130) (width 0.2) (layer "F.Cu") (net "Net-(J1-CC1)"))
 (via (at 225 130) (size 0.6) (drill 0.3) (layers "F.Cu" "B.Cu") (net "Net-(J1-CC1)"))
 (segment (start 225 130) (end 224.54 130) (width 0.2) (layer "B.Cu") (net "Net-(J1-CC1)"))
 (segment (start 224.54 130) (end 215.165 120.625) (width 0.2) (layer "B.Cu") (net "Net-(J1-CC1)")))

